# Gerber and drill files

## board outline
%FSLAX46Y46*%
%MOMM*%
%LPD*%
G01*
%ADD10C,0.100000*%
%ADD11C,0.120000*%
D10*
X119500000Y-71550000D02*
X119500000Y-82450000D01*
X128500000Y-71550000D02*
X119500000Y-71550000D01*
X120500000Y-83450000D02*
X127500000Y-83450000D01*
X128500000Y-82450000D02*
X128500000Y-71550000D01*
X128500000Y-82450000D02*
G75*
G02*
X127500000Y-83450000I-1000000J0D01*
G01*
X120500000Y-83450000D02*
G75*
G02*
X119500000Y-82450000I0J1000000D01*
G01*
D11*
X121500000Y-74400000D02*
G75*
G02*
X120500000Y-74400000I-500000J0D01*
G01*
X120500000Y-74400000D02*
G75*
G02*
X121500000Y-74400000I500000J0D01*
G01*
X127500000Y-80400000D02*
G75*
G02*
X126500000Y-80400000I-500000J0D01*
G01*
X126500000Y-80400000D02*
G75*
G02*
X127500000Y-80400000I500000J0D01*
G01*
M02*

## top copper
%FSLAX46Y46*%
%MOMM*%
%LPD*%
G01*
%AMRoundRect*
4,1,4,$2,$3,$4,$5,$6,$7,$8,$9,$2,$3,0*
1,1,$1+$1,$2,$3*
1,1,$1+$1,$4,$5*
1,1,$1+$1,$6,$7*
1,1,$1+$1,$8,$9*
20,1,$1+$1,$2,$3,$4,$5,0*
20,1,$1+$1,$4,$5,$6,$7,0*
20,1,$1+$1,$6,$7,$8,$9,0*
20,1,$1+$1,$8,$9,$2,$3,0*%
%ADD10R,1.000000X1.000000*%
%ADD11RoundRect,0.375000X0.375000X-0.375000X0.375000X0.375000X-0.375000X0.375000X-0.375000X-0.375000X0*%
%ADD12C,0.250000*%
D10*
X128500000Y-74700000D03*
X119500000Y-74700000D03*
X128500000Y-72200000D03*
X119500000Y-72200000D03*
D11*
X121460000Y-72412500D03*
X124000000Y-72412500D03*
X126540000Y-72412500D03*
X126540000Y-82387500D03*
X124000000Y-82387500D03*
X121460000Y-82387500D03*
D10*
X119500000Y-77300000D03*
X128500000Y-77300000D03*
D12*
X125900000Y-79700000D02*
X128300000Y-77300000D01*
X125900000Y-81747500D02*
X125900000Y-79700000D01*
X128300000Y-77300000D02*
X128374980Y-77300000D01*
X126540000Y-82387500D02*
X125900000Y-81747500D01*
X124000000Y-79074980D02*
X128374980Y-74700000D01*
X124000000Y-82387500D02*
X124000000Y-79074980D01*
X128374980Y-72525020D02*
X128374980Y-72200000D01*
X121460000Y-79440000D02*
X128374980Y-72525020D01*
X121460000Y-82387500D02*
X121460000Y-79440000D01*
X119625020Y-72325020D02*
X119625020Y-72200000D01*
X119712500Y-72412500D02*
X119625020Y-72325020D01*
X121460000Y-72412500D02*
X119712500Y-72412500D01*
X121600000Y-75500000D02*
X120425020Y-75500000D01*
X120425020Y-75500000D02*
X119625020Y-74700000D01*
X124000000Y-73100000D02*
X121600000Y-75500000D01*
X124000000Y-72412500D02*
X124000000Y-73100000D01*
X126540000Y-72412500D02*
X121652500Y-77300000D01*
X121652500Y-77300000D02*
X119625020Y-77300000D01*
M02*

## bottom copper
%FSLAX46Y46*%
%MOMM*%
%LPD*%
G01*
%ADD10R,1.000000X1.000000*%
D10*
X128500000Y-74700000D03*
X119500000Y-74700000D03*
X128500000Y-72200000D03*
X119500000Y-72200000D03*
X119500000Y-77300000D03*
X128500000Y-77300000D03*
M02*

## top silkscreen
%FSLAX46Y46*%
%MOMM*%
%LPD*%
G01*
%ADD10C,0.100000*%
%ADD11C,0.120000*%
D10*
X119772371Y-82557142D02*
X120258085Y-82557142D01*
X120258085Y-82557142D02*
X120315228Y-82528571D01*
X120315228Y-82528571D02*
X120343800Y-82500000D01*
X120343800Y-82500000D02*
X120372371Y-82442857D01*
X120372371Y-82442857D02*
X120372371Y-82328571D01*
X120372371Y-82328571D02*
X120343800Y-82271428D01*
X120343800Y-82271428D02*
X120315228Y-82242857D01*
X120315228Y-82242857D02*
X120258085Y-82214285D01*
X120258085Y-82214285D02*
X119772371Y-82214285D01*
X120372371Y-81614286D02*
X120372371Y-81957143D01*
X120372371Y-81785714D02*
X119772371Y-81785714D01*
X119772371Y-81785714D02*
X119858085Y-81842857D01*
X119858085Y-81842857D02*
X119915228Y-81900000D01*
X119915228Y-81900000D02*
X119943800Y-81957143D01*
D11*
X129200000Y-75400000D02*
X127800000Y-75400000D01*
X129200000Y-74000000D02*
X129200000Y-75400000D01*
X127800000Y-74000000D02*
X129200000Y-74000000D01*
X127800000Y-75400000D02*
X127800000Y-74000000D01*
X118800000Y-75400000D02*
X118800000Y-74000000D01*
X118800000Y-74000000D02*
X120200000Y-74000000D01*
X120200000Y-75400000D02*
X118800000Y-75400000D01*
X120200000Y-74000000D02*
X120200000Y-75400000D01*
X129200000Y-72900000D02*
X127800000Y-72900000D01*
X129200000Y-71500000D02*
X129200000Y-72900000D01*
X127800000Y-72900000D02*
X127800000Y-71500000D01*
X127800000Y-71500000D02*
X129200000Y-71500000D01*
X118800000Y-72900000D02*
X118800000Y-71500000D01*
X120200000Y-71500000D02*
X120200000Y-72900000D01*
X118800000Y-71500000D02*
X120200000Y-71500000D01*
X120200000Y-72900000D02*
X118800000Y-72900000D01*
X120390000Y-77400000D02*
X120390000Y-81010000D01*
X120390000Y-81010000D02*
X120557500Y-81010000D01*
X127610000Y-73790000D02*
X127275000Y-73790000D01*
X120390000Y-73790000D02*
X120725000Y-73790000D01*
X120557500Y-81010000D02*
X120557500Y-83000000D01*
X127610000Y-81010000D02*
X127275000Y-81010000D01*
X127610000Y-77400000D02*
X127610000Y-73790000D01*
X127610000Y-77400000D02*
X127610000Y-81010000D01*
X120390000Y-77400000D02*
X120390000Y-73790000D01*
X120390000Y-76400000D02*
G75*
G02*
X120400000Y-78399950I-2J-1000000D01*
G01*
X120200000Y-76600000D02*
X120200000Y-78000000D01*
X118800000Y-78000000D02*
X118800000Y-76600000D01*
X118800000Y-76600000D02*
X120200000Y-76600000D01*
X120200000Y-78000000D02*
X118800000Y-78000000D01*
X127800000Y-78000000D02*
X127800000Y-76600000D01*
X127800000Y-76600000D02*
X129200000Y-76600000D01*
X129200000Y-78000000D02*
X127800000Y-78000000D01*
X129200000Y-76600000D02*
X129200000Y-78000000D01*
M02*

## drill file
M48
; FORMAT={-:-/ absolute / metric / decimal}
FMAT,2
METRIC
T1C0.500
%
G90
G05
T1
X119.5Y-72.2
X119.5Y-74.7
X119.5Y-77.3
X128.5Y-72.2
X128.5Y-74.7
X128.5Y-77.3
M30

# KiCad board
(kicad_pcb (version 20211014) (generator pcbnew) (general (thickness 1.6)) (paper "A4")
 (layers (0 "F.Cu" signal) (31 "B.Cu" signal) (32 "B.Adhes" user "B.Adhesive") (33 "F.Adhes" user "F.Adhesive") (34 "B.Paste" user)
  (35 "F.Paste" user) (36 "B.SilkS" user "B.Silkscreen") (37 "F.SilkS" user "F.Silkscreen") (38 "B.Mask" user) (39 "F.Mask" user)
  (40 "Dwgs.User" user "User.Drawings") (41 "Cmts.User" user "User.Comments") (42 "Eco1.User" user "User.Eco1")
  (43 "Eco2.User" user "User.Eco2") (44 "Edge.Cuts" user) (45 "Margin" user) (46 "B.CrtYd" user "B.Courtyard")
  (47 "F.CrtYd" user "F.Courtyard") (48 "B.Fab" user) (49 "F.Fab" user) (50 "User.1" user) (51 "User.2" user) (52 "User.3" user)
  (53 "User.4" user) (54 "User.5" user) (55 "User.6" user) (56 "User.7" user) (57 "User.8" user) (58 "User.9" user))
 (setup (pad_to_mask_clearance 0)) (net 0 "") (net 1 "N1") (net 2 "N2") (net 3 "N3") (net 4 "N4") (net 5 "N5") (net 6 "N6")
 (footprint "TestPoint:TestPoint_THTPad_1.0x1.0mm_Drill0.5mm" (layer "F.Cu") (at 128.5 74.7)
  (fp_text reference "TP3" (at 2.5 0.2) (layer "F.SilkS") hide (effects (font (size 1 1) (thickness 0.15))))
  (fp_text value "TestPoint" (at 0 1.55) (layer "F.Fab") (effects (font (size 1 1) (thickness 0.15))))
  (fp_line (start 0.7 0.7) (end -0.7 0.7) (layer "F.SilkS") (width 0.12))
  (fp_line (start 0.7 -0.7) (end 0.7 0.7) (layer "F.SilkS") (width 0.12))
  (fp_line (start -0.7 -0.7) (end 0.7 -0.7) (layer "F.SilkS") (width 0.12))
  (fp_line (start -0.7 0.7) (end -0.7 -0.7) (layer "F.SilkS") (width 0.12))
  (pad "1" thru_hole rect (at 0 0) (size 1 1) (drill 0.5) (layers *.Cu *.Mask) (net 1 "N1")))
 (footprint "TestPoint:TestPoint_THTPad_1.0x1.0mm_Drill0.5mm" (layer "F.Cu") (at 119.5 74.7)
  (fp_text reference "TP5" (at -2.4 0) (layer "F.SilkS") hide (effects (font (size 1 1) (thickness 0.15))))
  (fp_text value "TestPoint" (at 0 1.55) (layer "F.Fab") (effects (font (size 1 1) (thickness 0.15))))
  (fp_line (start -0.7 0.7) (end -0.7 -0.7) (layer "F.SilkS") (width 0.12))
  (fp_line (start -0.7 -0.7) (end 0.7 -0.7) (layer "F.SilkS") (width 0.12))
  (fp_line (start 0.7 0.7) (end -0.7 0.7) (layer "F.SilkS") (width 0.12))
  (fp_line (start 0.7 -0.7) (end 0.7 0.7) (layer "F.SilkS") (width 0.12))
  (pad "1" thru_hole rect (at 0 0) (size 1 1) (drill 0.5) (layers *.Cu *.Mask) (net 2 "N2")))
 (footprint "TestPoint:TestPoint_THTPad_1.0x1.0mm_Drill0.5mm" (layer "F.Cu") (at 128.5 72.2)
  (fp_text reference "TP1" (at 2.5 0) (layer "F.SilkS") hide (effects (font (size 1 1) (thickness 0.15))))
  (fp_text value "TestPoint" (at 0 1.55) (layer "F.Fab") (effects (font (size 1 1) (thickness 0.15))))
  (fp_line (start 0.7 0.7) (end -0.7 0.7) (layer "F.SilkS") (width 0.12))
  (fp_line (start 0.7 -0.7) (end 0.7 0.7) (layer "F.SilkS") (width 0.12))
  (fp_line (start -0.7 0.7) (end -0.7 -0.7) (layer "F.SilkS") (width 0.12))
  (fp_line (start -0.7 -0.7) (end 0.7 -0.7) (layer "F.SilkS") (width 0.12))
  (pad "1" thru_hole rect (at 0 0) (size 1 1) (drill 0.5) (layers *.Cu *.Mask) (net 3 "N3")))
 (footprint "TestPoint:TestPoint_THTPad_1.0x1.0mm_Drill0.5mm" (layer "F.Cu") (at 119.5 72.2)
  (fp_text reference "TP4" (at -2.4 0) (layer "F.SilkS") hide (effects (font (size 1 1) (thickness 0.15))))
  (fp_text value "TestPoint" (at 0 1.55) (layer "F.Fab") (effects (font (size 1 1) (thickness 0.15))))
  (fp_line (start -0.7 0.7) (end -0.7 -0.7) (layer "F.SilkS") (width 0.12))
  (fp_line (start 0.7 -0.7) (end 0.7 0.7) (layer "F.SilkS") (width 0.12))
  (fp_line (start -0.7 -0.7) (end 0.7 -0.7) (layer "F.SilkS") (width 0.12))
  (fp_line (start 0.7 0.7) (end -0.7 0.7) (layer "F.SilkS") (width 0.12))
  (pad "1" thru_hole rect (at 0 0) (size 1 1) (drill 0.5) (layers *.Cu *.Mask) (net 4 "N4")))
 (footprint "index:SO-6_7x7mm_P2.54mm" (layer "F.Cu") (at 124 77.4 90)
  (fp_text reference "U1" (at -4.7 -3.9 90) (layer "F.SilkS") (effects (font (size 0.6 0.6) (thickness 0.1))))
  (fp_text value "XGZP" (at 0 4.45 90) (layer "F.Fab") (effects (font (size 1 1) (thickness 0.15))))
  (fp_line (start 0 -3.61) (end -3.61 -3.61) (layer "F.SilkS") (width 0.12))
  (fp_line (start -3.61 -3.61) (end -3.61 -3.4425) (layer "F.SilkS") (width 0.12))
  (fp_line (start 3.61 3.61) (end 3.61 3.275) (layer "F.SilkS") (width 0.12))
  (fp_line (start 3.61 -3.61) (end 3.61 -3.275) (layer "F.SilkS") (width 0.12))
  (fp_line (start -3.61 -3.4425) (end -5.6 -3.4425) (layer "F.SilkS") (width 0.12))
  (fp_line (start -3.61 3.61) (end -3.61 3.275) (layer "F.SilkS") (width 0.12))
  (fp_line (start 0 3.61) (end 3.61 3.61) (layer "F.SilkS") (width 0.12))
  (fp_line (start 0 3.61) (end -3.61 3.61) (layer "F.SilkS") (width 0.12))
  (fp_line (start 0 -3.61) (end 3.61 -3.61) (layer "F.SilkS") (width 0.12))
  (fp_arc (start 1 -3.61) (mid 0.005 -2.610014) (end -0.99995 -3.6) (layer "F.SilkS") (width 0.12))
  (fp_circle (center 3 -3) (end 3.5 -3) (layer "Edge.Cuts") (width 0.12) (fill none))
  (fp_circle (center -3 3) (end -2.5 3) (layer "Edge.Cuts") (width 0.12) (fill none))
  (pad "1" smd roundrect (at 4.9875 -2.54 90) (size 1.5 1.5) (layers "F.Cu" "F.Paste" "F.Mask") (roundrect_rratio 0.25) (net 4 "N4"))
  (pad "2" smd roundrect (at 4.9875 0 90) (size 1.5 1.5) (layers "F.Cu" "F.Paste" "F.Mask") (roundrect_rratio 0.25) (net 2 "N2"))
  (pad "3" smd roundrect (at 4.9875 2.54 90) (size 1.5 1.5) (layers "F.Cu" "F.Paste" "F.Mask") (roundrect_rratio 0.25) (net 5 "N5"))
  (pad "4" smd roundrect (at -4.9875 2.54 90) (size 1.5 1.5) (layers "F.Cu" "F.Paste" "F.Mask") (roundrect_rratio 0.25) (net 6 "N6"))
  (pad "5" smd roundrect (at -4.9875 0 90) (size 1.5 1.5) (layers "F.Cu" "F.Paste" "F.Mask") (roundrect_rratio 0.25) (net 1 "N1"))
  (pad "6" smd roundrect (at -4.9875 -2.54 90) (size 1.5 1.5) (layers "F.Cu" "F.Paste" "F.Mask") (roundrect_rratio 0.25) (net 3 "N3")))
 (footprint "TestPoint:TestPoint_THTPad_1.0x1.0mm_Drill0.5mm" (layer "F.Cu") (at 119.5 77.3)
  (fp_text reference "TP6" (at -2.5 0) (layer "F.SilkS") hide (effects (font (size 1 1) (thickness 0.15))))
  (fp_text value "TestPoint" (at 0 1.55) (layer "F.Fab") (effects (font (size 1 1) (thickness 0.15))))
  (fp_line (start 0.7 -0.7) (end 0.7 0.7) (layer "F.SilkS") (width 0.12))
  (fp_line (start -0.7 0.7) (end -0.7 -0.7) (layer "F.SilkS") (width 0.12))
  (fp_line (start -0.7 -0.7) (end 0.7 -0.7) (layer "F.SilkS") (width 0.12))
  (fp_line (start 0.7 0.7) (end -0.7 0.7) (layer "F.SilkS") (width 0.12))
  (pad "1" thru_hole rect (at 0 0) (size 1 1) (drill 0.5) (layers *.Cu *.Mask) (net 5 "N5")))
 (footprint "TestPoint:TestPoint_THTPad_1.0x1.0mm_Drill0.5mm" (layer "F.Cu") (at 128.5 77.3)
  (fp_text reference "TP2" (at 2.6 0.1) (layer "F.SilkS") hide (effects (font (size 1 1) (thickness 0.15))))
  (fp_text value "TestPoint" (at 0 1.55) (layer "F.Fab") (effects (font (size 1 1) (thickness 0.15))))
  (fp_line (start -0.7 0.7) (end -0.7 -0.7) (layer "F.SilkS") (width 0.12))
  (fp_line (start -0.7 -0.7) (end 0.7 -0.7) (layer "F.SilkS") (width 0.12))
  (fp_line (start 0.7 0.7) (end -0.7 0.7) (layer "F.SilkS") (width 0.12))
  (fp_line (start 0.7 -0.7) (end 0.7 0.7) (layer "F.SilkS") (width 0.12))
  (pad "1" thru_hole rect (at 0 0) (size 1 1) (drill 0.5) (layers *.Cu *.Mask) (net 6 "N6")))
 (gr_line (start 119.5 71.55) (end 119.5 82.45) (layer "Edge.Cuts") (width 0.1))
 (gr_line (start 128.5 71.55) (end 119.5 71.55) (layer "Edge.Cuts") (width 0.1))
 (gr_line (start 120.5 83.45) (end 127.5 83.45) (layer "Edge.Cuts") (width 0.1))
 (gr_line (start 128.5 82.45) (end 128.5 71.55) (layer "Edge.Cuts") (width 0.1))
 (gr_arc (start 128.5 82.45) (mid 128.207107 83.157107) (end 127.5 83.45) (layer "Edge.Cuts") (width 0.1))
 (gr_arc (start 120.5 83.45) (mid 119.792893 83.157107) (end 119.5 82.45) (layer "Edge.Cuts") (width 0.1))
 (segment (start 125.9 79.7) (end 128.3 77.3) (width 0.25) (layer "F.Cu") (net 6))
 (segment (start 125.9 81.7475) (end 125.9 79.7) (width 0.25) (layer "F.Cu") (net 6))
 (segment (start 128.3 77.3) (end 128.37498 77.3) (width 0.25) (layer "F.Cu") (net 6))
 (segment (start 126.54 82.3875) (end 125.9 81.7475) (width 0.25) (layer "F.Cu") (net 6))
 (segment (start 124 79.07498) (end 128.37498 74.7) (width 0.25) (layer "F.Cu") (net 1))
 (segment (start 124 82.3875) (end 124 79.07498) (width 0.25) (layer "F.Cu") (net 1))
 (segment (start 128.37498 72.52502) (end 128.37498 72.2) (width 0.25) (layer "F.Cu") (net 3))
 (segment (start 121.46 79.44) (end 128.37498 72.52502) (width 0.25) (layer "F.Cu") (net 3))
 (segment (start 121.46 82.3875) (end 121.46 79.44) (width 0.25) (layer "F.Cu") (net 3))
 (segment (start 119.62502 72.32502) (end 119.62502 72.2) (width 0.25) (layer "F.Cu") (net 4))
 (segment (start 119.7125 72.4125) (end 119.62502 72.32502) (width 0.25) (layer "F.Cu") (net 4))
 (segment (start 121.46 72.4125) (end 119.7125 72.4125) (width 0.25) (layer "F.Cu") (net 4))
 (segment (start 121.6 75.5) (end 120.42502 75.5) (width 0.25) (layer "F.Cu") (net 2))
 (segment (start 120.42502 75.5) (end 119.62502 74.7) (width 0.25) (layer "F.Cu") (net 2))
 (segment (start 124 73.1) (end 121.6 75.5) (width 0.25) (layer "F.Cu") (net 2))
 (segment (start 124 72.4125) (end 124 73.1) (width 0.25) (layer "F.Cu") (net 2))
 (segment (start 126.54 72.4125) (end 121.6525 77.3) (width 0.25) (layer "F.Cu") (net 5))
 (segment (start 121.6525 77.3) (end 119.62502 77.3) (width 0.25) (layer "F.Cu") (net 5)))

